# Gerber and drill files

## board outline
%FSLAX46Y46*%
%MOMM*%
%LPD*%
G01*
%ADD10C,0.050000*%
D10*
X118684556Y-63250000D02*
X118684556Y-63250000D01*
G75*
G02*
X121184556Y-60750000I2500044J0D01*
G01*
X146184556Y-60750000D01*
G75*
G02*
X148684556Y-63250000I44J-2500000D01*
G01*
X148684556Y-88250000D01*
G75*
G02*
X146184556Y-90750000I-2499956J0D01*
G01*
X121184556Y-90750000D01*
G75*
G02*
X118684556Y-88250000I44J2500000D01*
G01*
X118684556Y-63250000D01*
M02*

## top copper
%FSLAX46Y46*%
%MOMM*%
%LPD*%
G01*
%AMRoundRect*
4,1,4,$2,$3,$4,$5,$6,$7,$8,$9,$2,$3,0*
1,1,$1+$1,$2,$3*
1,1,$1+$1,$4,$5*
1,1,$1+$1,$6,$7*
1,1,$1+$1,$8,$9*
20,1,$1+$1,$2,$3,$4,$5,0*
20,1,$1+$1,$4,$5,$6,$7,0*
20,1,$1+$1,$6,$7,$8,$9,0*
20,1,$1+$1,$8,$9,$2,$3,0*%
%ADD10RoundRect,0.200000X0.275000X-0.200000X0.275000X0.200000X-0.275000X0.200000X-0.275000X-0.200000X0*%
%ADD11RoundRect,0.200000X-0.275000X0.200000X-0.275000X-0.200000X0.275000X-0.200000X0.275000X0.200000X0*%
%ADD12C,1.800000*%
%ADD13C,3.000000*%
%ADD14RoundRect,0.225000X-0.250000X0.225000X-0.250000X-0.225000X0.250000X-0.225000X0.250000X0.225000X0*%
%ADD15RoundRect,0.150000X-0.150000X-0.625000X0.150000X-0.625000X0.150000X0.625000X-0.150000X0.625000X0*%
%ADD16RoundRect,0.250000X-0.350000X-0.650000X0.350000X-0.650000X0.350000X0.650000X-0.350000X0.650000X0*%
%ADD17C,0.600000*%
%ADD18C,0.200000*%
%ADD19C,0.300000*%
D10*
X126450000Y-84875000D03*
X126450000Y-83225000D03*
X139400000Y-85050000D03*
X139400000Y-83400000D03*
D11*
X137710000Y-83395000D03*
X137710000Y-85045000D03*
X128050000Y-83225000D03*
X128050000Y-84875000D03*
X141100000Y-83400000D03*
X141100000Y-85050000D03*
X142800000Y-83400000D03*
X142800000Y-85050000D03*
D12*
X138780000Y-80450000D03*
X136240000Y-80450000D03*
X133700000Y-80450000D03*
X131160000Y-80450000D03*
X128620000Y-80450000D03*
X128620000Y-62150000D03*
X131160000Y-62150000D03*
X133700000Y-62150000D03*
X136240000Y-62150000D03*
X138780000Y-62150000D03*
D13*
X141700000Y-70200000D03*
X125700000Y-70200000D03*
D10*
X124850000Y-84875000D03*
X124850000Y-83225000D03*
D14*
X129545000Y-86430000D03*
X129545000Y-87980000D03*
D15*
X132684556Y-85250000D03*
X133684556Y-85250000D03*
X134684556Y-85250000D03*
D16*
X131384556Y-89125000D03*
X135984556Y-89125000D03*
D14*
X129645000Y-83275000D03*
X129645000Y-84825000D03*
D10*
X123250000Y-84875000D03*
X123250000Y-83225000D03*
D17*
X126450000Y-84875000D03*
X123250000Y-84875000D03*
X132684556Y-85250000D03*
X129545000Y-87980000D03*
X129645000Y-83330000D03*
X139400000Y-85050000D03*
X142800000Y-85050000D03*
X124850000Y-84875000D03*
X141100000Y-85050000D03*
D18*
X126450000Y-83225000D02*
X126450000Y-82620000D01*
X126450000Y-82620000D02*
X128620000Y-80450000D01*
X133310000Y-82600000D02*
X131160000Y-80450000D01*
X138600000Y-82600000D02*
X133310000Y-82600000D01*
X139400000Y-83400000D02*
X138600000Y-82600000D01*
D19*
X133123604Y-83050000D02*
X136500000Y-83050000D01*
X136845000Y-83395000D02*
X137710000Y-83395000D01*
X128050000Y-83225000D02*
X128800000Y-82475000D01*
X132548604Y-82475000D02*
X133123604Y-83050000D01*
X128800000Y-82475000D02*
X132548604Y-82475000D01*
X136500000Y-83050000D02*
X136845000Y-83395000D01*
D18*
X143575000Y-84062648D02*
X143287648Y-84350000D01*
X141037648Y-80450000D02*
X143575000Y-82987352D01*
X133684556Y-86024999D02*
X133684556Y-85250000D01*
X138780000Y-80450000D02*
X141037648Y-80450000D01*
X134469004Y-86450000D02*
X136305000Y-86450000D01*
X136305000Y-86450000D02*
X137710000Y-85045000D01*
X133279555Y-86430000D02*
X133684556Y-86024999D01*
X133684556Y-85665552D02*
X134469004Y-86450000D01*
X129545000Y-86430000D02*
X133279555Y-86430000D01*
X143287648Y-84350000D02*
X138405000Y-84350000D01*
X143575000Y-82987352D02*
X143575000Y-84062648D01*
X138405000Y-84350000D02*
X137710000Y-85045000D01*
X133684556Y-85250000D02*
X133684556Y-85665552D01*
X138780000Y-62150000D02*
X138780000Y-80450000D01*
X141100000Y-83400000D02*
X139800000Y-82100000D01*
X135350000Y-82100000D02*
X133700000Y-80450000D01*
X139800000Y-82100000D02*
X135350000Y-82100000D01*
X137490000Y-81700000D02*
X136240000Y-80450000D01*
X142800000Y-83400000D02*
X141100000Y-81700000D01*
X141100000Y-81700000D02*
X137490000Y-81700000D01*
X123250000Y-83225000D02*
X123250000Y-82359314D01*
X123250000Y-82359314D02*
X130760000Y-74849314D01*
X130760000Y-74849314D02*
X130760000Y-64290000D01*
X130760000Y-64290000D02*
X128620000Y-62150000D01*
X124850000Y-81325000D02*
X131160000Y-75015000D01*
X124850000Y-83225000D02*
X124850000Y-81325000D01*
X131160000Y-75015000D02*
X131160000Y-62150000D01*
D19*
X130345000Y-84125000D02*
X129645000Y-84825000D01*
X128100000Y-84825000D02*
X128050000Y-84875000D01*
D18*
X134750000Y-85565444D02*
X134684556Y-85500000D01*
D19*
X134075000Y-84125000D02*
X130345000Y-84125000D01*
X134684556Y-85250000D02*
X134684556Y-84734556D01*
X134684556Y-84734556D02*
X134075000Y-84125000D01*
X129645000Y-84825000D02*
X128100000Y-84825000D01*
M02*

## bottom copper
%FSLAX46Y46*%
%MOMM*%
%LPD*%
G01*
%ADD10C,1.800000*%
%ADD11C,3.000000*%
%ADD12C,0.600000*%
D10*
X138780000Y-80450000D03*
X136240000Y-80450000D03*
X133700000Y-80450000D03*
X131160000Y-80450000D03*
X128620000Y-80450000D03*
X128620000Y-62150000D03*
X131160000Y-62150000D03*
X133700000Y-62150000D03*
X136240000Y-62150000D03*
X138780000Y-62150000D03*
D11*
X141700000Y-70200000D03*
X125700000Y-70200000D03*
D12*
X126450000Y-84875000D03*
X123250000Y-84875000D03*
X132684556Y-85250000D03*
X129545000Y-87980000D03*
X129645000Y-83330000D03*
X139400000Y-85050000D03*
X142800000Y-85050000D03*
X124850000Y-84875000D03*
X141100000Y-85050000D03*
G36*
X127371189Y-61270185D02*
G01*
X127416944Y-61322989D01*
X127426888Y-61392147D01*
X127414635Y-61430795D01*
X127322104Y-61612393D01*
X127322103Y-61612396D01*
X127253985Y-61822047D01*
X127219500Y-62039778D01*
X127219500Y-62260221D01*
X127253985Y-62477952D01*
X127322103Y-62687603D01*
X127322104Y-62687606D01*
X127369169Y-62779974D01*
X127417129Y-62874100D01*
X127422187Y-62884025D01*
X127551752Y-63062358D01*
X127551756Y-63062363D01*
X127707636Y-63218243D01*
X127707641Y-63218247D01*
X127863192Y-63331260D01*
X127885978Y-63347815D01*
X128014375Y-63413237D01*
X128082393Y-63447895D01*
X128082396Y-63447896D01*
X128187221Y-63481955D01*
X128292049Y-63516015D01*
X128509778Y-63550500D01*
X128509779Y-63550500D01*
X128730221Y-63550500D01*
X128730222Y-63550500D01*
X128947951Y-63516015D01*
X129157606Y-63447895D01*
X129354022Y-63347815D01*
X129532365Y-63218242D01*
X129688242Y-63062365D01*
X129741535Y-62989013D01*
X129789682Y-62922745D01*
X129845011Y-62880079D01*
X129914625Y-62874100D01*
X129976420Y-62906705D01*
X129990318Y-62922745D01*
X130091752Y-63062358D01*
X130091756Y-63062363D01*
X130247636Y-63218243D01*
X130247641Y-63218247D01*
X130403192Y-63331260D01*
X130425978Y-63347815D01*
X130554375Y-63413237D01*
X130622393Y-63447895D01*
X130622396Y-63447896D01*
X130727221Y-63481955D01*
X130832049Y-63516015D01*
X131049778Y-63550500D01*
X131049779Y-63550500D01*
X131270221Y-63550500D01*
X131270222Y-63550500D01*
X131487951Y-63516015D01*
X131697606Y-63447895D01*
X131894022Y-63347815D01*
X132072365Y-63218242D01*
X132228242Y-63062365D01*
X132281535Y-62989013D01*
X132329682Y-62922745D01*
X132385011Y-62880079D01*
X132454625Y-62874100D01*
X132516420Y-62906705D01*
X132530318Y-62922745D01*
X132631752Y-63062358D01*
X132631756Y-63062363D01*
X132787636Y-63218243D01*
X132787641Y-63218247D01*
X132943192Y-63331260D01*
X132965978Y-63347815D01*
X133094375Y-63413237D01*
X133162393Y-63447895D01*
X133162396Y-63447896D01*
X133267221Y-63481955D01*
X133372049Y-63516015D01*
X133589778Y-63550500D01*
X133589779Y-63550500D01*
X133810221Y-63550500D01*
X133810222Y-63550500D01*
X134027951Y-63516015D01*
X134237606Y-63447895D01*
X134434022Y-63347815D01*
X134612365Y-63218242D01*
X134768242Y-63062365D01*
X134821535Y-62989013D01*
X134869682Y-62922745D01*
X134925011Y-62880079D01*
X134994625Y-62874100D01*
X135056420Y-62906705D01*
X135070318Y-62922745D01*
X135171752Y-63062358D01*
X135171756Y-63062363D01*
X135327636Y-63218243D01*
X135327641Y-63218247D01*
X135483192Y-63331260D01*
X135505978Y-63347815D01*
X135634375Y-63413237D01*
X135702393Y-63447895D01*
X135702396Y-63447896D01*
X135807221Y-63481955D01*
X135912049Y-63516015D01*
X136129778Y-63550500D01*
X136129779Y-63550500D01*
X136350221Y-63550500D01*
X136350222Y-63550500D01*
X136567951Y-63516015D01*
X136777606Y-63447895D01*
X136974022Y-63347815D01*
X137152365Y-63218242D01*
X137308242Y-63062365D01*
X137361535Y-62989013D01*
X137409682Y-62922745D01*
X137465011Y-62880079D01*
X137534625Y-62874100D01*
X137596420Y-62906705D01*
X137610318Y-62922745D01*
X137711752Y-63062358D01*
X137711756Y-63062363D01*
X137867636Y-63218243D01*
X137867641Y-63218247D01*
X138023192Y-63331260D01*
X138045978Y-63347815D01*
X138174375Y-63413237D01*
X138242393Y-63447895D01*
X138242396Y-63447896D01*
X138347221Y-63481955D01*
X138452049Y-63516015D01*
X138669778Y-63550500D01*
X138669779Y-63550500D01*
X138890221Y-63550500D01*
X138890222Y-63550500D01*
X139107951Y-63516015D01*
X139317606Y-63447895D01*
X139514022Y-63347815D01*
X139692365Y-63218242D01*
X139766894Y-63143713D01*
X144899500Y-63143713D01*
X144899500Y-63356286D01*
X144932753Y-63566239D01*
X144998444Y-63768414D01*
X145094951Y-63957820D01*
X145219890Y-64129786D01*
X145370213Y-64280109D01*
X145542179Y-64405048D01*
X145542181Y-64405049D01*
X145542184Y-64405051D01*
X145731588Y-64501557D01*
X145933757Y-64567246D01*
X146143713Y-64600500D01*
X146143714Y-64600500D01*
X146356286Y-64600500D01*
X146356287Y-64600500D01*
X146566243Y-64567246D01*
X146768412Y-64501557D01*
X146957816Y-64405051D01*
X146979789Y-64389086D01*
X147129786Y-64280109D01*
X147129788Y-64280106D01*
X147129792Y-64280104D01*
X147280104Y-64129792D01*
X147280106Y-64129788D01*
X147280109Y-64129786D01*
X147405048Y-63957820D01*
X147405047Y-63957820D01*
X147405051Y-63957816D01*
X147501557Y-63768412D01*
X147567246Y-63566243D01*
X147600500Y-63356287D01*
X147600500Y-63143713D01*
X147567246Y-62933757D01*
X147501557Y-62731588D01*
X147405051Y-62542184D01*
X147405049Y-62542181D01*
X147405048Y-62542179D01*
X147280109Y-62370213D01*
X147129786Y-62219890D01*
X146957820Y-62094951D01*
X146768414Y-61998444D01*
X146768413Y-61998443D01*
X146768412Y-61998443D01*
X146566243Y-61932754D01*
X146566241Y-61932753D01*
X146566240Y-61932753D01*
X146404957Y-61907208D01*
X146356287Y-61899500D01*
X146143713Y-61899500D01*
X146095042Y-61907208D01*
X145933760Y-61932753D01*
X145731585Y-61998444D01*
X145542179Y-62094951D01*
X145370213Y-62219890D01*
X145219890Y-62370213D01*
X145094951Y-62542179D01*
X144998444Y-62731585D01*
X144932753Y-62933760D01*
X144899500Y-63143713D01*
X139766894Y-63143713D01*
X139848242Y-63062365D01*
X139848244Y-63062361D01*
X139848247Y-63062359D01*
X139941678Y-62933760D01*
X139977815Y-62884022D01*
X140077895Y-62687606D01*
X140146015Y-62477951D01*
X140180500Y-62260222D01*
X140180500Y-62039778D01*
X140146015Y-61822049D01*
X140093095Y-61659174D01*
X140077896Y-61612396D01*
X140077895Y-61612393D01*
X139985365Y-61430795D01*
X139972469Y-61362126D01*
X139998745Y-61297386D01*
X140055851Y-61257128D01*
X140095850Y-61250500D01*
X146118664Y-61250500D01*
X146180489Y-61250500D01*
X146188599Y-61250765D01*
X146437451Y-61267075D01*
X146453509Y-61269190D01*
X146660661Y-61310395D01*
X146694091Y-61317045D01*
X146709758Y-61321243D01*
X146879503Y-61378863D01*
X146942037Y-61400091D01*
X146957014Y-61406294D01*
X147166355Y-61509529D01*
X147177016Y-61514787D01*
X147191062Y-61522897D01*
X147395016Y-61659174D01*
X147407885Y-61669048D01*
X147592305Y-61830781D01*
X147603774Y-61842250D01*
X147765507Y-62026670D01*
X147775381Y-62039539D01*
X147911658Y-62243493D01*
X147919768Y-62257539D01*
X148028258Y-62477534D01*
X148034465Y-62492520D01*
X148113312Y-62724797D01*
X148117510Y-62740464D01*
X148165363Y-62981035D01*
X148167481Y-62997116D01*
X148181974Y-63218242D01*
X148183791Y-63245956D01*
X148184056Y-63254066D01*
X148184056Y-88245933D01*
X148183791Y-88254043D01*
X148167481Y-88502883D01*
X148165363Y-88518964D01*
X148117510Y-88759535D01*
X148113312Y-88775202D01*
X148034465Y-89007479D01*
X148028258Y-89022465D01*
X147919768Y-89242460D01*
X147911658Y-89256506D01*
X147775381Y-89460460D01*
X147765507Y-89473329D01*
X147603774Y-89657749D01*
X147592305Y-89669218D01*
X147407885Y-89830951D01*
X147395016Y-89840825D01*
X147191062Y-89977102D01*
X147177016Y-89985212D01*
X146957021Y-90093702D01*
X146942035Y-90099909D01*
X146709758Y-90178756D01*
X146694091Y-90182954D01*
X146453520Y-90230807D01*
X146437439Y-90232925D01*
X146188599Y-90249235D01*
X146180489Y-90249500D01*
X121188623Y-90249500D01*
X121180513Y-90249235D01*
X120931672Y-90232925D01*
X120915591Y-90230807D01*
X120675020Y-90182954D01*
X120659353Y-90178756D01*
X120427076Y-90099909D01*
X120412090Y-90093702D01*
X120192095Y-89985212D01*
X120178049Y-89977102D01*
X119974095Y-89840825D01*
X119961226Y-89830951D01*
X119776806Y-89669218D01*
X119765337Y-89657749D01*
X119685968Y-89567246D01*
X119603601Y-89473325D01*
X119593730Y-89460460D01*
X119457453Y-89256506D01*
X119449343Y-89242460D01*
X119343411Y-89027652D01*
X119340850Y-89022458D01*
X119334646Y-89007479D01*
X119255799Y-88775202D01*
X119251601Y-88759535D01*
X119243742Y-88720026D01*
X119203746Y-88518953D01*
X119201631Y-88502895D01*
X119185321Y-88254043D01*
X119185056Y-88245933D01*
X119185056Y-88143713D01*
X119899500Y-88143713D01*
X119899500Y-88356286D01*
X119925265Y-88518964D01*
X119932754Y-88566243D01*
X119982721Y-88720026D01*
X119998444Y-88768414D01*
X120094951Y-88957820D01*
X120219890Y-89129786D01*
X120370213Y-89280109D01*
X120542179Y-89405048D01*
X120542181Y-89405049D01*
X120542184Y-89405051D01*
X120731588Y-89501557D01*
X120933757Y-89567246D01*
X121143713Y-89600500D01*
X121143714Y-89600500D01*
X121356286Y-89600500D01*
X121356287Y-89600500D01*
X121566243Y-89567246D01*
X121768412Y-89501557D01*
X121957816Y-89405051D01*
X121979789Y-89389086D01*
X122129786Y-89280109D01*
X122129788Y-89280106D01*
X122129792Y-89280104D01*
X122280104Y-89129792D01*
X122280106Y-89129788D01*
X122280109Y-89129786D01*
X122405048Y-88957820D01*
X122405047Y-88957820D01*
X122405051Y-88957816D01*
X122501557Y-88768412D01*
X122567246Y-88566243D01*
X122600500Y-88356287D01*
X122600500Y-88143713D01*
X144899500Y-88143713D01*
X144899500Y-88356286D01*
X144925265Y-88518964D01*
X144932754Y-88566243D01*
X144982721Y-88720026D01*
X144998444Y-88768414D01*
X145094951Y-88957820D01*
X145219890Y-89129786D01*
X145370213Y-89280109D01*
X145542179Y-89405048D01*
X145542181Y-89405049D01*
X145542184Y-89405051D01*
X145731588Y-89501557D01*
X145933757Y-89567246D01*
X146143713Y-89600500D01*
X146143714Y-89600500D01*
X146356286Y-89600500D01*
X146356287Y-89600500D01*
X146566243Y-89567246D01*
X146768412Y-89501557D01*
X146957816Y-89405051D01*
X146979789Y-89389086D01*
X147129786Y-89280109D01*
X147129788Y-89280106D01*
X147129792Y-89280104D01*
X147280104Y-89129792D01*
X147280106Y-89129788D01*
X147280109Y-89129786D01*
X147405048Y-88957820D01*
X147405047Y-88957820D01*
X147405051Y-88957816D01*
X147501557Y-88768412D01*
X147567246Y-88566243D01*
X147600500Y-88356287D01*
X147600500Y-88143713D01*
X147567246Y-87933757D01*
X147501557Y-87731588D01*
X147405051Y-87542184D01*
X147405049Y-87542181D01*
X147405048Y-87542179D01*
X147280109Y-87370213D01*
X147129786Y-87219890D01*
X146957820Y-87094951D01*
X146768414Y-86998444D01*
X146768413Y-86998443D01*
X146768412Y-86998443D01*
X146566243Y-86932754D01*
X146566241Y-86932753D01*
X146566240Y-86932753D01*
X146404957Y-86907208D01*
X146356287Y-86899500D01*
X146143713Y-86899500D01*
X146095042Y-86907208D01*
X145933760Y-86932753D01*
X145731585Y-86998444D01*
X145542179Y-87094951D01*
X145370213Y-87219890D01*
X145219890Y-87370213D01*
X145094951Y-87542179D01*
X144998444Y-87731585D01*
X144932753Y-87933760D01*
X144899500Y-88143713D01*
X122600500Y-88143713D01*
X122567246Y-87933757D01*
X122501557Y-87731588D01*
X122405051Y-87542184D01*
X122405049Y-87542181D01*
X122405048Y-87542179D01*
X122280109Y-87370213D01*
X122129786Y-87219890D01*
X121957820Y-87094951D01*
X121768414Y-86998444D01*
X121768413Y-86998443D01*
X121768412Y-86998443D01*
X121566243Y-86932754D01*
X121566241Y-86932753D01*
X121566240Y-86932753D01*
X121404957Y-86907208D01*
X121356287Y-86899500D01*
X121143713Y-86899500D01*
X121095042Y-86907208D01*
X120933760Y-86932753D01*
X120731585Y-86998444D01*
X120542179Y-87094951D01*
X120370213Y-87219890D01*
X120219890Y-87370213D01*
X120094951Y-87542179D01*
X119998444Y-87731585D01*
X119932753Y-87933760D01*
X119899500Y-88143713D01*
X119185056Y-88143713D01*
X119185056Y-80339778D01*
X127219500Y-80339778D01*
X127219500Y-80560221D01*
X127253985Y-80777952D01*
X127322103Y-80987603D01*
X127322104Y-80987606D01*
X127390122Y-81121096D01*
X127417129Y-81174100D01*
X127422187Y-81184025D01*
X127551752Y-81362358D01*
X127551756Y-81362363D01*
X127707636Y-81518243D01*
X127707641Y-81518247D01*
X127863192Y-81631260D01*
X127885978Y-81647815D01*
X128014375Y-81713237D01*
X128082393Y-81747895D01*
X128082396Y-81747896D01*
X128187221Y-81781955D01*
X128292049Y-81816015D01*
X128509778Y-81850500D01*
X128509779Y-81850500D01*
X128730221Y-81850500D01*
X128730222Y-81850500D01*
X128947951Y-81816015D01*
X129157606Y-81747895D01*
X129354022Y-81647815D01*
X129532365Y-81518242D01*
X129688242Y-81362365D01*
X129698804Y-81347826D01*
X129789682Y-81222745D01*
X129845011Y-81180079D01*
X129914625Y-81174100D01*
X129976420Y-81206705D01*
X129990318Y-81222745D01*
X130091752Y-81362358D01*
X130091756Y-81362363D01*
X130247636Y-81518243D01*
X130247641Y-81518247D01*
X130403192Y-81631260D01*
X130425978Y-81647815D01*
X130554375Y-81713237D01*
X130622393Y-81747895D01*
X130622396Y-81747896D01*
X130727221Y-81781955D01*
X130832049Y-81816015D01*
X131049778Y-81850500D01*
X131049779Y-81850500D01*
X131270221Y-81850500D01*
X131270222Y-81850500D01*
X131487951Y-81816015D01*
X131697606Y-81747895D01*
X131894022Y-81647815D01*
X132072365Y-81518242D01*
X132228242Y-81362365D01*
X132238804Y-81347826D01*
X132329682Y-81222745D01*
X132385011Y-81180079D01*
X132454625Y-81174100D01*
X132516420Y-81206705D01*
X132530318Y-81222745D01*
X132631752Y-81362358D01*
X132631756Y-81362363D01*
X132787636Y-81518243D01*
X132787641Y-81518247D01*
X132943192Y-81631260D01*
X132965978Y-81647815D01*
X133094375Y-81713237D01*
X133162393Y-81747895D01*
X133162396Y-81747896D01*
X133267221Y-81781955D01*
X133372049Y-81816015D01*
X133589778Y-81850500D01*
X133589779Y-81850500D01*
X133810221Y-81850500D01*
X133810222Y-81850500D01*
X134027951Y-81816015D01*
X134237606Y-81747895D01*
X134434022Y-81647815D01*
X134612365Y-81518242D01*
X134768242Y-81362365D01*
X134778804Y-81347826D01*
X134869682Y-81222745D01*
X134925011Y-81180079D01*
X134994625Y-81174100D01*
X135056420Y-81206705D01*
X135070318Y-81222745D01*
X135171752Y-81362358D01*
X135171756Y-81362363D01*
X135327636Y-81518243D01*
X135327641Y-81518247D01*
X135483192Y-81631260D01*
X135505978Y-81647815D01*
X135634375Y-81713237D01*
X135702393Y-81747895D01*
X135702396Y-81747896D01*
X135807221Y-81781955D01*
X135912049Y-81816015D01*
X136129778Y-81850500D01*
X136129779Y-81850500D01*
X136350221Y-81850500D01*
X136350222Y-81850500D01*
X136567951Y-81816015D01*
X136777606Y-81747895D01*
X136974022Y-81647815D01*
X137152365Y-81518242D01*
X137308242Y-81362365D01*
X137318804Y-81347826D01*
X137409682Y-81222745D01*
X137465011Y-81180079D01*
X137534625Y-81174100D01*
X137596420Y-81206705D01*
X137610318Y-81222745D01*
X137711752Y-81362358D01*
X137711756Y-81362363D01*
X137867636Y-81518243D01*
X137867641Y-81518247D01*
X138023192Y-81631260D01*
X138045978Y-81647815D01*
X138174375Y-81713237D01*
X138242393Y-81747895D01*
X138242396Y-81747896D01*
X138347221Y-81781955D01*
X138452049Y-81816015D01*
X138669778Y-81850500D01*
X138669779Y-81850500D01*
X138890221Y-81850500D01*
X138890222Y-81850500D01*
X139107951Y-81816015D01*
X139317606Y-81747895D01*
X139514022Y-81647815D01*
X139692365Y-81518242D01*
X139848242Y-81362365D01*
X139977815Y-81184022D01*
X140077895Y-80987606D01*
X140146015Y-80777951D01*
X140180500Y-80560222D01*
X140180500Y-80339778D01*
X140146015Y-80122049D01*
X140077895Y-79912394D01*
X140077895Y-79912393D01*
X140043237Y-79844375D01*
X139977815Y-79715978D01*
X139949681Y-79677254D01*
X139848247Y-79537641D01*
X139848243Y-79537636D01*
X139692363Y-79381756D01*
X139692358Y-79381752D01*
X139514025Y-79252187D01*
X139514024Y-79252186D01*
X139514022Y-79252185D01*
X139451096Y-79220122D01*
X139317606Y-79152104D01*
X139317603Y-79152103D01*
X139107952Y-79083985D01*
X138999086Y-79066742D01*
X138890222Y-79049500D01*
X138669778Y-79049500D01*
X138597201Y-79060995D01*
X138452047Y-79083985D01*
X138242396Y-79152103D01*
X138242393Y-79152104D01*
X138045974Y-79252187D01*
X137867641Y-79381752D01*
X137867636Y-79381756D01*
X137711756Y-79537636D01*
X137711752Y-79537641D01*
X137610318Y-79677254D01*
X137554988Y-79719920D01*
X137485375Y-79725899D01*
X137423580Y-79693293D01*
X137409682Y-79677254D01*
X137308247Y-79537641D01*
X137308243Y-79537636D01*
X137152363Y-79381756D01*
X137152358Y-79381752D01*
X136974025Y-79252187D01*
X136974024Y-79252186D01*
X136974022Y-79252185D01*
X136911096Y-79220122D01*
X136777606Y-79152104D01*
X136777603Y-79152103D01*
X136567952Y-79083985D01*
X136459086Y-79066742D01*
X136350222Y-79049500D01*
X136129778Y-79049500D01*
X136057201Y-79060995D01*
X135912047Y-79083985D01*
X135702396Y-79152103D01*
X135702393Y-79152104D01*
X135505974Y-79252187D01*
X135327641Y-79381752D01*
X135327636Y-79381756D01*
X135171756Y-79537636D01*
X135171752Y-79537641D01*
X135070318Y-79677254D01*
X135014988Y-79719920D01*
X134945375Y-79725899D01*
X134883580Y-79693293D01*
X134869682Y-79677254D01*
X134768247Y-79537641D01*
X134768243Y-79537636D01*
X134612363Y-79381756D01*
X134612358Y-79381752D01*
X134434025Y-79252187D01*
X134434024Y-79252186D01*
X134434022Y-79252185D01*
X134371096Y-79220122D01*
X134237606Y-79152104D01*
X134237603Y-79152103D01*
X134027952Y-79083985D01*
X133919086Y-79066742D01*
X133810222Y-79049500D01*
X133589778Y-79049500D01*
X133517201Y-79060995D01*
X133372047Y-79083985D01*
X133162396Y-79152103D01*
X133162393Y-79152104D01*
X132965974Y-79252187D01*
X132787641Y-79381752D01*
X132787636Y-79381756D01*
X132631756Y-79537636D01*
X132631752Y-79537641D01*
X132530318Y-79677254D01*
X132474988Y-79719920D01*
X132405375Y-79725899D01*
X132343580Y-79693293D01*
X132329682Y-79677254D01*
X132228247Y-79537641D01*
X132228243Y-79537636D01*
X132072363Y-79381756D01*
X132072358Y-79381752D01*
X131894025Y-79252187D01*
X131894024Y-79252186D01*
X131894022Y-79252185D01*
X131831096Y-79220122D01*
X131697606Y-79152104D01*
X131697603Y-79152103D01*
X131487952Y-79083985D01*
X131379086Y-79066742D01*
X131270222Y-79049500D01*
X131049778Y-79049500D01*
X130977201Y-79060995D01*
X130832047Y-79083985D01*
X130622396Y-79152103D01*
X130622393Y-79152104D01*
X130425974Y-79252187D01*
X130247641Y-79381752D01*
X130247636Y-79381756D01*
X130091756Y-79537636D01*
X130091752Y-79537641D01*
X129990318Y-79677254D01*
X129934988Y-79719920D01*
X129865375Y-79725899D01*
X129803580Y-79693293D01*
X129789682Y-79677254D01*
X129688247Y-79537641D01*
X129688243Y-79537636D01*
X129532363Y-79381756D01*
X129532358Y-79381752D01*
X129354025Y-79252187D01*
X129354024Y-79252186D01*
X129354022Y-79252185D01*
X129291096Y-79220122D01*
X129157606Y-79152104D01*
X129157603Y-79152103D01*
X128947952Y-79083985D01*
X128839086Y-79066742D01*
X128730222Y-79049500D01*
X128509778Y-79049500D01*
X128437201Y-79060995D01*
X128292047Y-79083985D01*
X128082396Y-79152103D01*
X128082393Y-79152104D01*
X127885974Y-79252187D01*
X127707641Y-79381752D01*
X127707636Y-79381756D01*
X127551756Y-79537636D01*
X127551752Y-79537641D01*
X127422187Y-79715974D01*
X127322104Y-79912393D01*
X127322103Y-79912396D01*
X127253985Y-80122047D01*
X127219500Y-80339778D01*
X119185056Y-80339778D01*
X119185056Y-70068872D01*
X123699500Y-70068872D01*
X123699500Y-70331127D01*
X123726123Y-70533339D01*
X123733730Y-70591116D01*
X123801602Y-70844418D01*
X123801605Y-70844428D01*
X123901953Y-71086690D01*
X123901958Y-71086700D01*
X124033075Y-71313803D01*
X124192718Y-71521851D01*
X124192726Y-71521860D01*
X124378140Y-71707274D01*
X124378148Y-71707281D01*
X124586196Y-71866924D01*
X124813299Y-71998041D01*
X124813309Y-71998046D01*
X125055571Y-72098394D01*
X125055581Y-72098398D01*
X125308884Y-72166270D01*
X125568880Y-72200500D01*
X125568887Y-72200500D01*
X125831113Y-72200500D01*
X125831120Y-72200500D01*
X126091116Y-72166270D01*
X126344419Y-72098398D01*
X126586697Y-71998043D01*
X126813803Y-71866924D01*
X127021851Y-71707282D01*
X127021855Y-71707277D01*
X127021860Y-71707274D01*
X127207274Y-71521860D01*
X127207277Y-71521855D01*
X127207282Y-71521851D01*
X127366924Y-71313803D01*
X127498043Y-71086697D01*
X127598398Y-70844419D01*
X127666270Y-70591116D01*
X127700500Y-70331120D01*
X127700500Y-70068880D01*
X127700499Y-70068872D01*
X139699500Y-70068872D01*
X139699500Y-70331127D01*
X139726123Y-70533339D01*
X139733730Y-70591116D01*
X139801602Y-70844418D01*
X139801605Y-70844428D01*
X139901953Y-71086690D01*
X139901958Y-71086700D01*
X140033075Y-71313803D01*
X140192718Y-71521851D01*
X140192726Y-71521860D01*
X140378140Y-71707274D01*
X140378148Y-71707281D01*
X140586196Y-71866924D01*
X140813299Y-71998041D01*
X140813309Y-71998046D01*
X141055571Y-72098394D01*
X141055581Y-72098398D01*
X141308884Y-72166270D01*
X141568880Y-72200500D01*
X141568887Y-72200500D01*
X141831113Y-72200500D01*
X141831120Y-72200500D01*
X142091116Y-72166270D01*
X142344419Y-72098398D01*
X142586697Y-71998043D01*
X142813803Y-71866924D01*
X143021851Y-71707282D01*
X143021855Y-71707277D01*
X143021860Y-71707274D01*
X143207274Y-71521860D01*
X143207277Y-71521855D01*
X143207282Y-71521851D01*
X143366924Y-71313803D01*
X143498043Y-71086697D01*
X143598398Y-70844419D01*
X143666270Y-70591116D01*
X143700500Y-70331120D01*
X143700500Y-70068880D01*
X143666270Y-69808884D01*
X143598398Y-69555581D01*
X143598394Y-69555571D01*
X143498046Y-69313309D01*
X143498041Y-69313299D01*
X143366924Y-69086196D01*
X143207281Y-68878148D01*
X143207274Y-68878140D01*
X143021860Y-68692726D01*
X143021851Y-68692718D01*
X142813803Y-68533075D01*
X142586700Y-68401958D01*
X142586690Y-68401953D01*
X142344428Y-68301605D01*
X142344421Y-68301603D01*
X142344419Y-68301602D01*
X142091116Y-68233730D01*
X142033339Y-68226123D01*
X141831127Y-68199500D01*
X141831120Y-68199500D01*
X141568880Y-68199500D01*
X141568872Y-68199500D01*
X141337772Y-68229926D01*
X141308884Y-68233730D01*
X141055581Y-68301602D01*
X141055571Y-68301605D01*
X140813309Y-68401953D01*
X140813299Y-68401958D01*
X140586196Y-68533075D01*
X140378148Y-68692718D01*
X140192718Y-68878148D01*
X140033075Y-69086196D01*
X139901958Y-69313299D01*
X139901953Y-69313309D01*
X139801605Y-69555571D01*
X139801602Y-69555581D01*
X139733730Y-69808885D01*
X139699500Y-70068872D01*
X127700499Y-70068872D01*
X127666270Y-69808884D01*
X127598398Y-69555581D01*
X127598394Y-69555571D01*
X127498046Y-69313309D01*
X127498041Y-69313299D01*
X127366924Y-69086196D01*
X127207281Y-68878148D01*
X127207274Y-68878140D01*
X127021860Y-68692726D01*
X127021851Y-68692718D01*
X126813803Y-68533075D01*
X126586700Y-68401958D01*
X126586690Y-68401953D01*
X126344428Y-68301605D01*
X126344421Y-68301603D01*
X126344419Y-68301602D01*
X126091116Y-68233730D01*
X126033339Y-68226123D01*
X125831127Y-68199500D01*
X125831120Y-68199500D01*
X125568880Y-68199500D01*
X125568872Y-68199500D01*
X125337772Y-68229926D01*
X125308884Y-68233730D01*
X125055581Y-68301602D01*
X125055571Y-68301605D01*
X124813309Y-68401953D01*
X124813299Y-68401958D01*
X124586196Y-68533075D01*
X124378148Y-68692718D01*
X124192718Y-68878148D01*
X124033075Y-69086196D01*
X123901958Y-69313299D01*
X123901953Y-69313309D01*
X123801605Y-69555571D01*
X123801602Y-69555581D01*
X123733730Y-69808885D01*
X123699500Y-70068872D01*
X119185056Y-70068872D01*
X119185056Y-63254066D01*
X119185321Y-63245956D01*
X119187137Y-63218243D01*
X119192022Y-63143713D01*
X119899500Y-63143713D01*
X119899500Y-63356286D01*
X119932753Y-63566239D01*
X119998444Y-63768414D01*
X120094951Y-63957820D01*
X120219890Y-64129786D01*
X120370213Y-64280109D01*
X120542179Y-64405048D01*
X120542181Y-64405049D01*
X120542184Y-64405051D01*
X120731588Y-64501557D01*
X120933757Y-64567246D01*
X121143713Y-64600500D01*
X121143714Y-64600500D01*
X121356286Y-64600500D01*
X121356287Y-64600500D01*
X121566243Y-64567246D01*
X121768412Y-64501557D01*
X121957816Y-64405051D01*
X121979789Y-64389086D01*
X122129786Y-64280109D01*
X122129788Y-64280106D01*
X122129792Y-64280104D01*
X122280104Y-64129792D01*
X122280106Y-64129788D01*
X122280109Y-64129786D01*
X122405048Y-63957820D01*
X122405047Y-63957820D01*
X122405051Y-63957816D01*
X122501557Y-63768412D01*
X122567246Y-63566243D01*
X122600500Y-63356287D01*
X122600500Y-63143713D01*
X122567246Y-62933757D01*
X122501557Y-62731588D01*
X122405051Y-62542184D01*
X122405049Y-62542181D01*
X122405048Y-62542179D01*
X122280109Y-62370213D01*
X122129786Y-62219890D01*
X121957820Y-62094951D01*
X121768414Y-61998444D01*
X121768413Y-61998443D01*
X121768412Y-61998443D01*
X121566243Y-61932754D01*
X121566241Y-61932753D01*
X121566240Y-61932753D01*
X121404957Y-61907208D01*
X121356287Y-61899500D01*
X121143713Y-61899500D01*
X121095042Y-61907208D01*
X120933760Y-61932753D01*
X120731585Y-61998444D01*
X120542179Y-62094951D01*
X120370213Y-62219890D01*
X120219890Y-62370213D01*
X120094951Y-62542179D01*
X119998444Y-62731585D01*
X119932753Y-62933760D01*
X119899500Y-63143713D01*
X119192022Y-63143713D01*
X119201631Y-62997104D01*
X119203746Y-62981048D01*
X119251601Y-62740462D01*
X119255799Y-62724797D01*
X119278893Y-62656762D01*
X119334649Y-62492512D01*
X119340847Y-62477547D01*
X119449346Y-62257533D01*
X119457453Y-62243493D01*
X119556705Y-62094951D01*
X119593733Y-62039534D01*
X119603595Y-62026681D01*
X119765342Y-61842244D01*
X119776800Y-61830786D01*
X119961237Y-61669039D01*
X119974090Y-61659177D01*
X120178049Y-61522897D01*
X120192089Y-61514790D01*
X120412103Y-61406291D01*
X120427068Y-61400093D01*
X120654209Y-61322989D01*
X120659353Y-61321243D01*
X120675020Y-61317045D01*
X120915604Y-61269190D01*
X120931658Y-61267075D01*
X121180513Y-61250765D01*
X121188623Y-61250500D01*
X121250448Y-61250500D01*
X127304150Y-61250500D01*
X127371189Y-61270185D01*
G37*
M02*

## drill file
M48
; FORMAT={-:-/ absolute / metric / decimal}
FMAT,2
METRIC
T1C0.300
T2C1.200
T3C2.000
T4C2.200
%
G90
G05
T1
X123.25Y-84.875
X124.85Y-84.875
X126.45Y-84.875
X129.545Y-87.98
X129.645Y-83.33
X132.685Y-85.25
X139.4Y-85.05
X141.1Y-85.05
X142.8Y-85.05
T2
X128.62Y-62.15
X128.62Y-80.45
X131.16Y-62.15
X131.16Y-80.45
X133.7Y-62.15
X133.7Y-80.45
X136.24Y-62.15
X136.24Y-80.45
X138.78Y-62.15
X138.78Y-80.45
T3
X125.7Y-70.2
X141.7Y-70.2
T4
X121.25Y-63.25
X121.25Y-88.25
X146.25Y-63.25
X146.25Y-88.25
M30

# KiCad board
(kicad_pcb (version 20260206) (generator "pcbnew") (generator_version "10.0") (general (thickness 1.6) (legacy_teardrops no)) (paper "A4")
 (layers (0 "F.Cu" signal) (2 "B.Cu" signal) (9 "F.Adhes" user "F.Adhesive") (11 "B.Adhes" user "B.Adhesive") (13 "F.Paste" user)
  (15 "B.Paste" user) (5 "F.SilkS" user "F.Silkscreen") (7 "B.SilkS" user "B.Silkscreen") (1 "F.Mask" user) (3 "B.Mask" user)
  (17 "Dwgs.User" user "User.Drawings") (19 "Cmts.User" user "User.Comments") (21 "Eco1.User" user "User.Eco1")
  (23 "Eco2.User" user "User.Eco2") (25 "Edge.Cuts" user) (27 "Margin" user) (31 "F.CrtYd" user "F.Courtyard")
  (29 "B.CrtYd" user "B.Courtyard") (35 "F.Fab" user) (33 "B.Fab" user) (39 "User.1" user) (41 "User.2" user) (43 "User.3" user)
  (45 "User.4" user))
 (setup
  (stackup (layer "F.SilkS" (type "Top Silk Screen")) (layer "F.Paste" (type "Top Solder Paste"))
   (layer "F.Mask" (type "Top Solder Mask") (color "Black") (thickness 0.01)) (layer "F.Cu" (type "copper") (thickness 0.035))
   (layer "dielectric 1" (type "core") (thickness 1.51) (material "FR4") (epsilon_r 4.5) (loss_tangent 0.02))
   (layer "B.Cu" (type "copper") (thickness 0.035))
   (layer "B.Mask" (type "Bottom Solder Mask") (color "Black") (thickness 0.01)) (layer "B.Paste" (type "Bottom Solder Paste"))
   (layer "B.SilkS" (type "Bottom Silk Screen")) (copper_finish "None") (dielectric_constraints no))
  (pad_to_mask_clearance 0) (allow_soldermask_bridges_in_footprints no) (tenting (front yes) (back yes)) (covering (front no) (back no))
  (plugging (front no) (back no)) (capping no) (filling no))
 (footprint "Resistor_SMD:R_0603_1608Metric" (layer "F.Cu") (at 126.45 84.05 90)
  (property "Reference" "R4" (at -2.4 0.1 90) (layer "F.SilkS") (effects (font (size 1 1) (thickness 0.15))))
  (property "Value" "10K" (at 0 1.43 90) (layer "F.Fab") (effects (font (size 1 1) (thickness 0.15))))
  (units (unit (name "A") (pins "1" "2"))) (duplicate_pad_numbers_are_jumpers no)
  (pad "1" smd roundrect (at -0.825 0 90) (size 0.8 0.95) (layers "F.Cu" "F.Mask" "F.Paste") (roundrect_rratio 0.25) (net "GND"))
  (pad "2" smd roundrect (at 0.825 0 90) (size 0.8 0.95) (layers "F.Cu" "F.Mask" "F.Paste") (roundrect_rratio 0.25) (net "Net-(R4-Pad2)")))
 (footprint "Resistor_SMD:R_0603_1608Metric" (layer "F.Cu") (at 139.4 84.225 90)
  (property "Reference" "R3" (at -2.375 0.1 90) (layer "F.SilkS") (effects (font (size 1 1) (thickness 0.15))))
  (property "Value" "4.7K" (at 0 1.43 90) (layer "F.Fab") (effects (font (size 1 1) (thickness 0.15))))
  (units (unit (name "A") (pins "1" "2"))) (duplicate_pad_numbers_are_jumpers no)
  (pad "1" smd roundrect (at -0.825 0 90) (size 0.8 0.95) (layers "F.Cu" "F.Mask" "F.Paste") (roundrect_rratio 0.25) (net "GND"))
  (pad "2" smd roundrect (at 0.825 0 90) (size 0.8 0.95) (layers "F.Cu" "F.Mask" "F.Paste") (roundrect_rratio 0.25) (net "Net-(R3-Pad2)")))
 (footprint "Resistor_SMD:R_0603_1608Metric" (layer "F.Cu") (at 137.71 84.22 -90)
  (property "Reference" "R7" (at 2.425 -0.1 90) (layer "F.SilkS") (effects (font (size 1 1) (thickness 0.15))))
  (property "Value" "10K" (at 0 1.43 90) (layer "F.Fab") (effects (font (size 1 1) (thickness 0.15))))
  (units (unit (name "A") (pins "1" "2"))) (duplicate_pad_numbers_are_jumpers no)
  (pad "1" smd roundrect (at -0.825 0 270) (size 0.8 0.95) (layers "F.Cu" "F.Mask" "F.Paste") (roundrect_rratio 0.25) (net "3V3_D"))
  (pad "2" smd roundrect (at 0.825 0 270) (size 0.8 0.95) (layers "F.Cu" "F.Mask" "F.Paste") (roundrect_rratio 0.25) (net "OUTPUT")))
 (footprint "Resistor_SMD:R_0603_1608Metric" (layer "F.Cu") (at 128.05 84.05 -90)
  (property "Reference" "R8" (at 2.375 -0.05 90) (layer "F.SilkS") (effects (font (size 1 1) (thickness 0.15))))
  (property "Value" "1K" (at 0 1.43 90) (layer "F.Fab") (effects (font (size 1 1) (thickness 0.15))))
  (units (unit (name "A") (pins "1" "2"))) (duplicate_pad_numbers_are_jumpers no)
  (pad "1" smd roundrect (at -0.825 0 270) (size 0.8 0.95) (layers "F.Cu" "F.Mask" "F.Paste") (roundrect_rratio 0.25) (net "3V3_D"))
  (pad "2" smd roundrect (at 0.825 0 270) (size 0.8 0.95) (layers "F.Cu" "F.Mask" "F.Paste") (roundrect_rratio 0.25) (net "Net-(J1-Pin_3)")))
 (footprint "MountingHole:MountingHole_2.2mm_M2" (layer "F.Cu") (at 146.25 63.25)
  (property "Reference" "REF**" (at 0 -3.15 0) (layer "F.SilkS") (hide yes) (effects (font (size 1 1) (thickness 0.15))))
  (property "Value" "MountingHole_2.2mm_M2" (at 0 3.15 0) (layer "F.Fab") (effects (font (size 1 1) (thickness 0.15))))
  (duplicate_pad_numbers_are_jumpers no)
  (pad "" np_thru_hole circle (at 0 0) (size 2.2 2.2) (drill 2.2) (layers "*.Cu" "*.Mask")))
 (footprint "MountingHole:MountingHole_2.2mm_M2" (layer "F.Cu") (at 146.25 88.25)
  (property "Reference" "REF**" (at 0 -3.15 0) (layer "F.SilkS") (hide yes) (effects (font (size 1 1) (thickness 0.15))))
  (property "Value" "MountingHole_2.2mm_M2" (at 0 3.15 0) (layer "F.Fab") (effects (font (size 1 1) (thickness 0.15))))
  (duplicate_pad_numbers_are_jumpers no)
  (pad "" np_thru_hole circle (at 0 0) (size 2.2 2.2) (drill 2.2) (layers "*.Cu" "*.Mask")))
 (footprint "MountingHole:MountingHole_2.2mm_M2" (layer "F.Cu") (at 121.25 88.25)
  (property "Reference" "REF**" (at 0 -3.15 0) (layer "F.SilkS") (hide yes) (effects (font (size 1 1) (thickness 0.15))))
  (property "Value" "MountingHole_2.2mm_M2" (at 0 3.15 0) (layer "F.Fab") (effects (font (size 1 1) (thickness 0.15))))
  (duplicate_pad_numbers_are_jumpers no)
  (pad "" np_thru_hole circle (at 0 0) (size 2.2 2.2) (drill 2.2) (layers "*.Cu" "*.Mask")))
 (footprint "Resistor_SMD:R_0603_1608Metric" (layer "F.Cu") (at 141.1 84.225 -90)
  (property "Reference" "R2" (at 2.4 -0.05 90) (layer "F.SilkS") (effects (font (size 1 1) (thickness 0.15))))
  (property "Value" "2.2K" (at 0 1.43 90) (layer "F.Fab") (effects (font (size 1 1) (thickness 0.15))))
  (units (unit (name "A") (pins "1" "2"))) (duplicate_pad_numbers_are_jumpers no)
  (pad "1" smd roundrect (at -0.825 0 270) (size 0.8 0.95) (layers "F.Cu" "F.Mask" "F.Paste") (roundrect_rratio 0.25) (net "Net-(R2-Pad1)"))
  (pad "2" smd roundrect (at 0.825 0 270) (size 0.8 0.95) (layers "F.Cu" "F.Mask" "F.Paste") (roundrect_rratio 0.25) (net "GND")))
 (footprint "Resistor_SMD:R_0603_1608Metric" (layer "F.Cu") (at 142.8 84.225 -90)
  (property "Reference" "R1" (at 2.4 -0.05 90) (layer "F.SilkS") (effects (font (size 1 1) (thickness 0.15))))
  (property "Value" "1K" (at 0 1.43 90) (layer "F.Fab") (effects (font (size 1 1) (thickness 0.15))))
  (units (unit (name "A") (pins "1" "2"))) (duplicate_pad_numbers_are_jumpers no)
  (pad "1" smd roundrect (at -0.825 0 270) (size 0.8 0.95) (layers "F.Cu" "F.Mask" "F.Paste") (roundrect_rratio 0.25) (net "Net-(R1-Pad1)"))
  (pad "2" smd roundrect (at 0.825 0 270) (size 0.8 0.95) (layers "F.Cu" "F.Mask" "F.Paste") (roundrect_rratio 0.25) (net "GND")))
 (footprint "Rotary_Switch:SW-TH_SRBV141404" (layer "F.Cu") (at 133.7 71.3)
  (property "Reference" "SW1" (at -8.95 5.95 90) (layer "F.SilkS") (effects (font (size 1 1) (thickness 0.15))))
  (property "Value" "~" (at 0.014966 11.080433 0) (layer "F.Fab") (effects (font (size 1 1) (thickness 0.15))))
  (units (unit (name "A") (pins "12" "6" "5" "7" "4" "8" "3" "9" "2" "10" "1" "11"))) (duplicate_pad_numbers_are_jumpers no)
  (pad "1" thru_hole circle (at 5.08 9.15) (size 1.8 1.8) (drill 1.2) (layers "*.Cu" "*.Mask") (remove_unused_layers no) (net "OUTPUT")
   (thermal_bridge_angle 90))
  (pad "2" thru_hole circle (at 2.54 9.15) (size 1.8 1.8) (drill 1.2) (layers "*.Cu" "*.Mask") (remove_unused_layers no)
   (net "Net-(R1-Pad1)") (thermal_bridge_angle 90))
  (pad "3" thru_hole circle (at 0 9.15) (size 1.8 1.8) (drill 1.2) (layers "*.Cu" "*.Mask") (remove_unused_layers no) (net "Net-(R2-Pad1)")
   (thermal_bridge_angle 90))
  (pad "4" thru_hole circle (at -2.54 9.15) (size 1.8 1.8) (drill 1.2) (layers "*.Cu" "*.Mask") (remove_unused_layers no)
   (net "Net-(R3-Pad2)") (thermal_bridge_angle 90))
  (pad "5" thru_hole circle (at -5.08 9.15) (size 1.8 1.8) (drill 1.2) (layers "*.Cu" "*.Mask") (remove_unused_layers no)
   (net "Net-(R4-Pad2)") (thermal_bridge_angle 90))
  (pad "6" thru_hole circle (at -5.08 -9.15) (size 1.8 1.8) (drill 1.2) (layers "*.Cu" "*.Mask") (remove_unused_layers no)
   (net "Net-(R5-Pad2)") (thermal_bridge_angle 90))
  (pad "7" thru_hole circle (at -2.54 -9.15) (size 1.8 1.8) (drill 1.2) (layers "*.Cu" "*.Mask") (remove_unused_layers no)
   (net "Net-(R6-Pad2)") (thermal_bridge_angle 90))
  (pad "8" thru_hole circle (at 0 -9.15) (size 1.8 1.8) (drill 1.2) (layers "*.Cu" "*.Mask") (remove_unused_layers no)
   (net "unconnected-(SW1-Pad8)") (thermal_bridge_angle 90))
  (pad "9" thru_hole circle (at 2.54 -9.15) (size 1.8 1.8) (drill 1.2) (layers "*.Cu" "*.Mask") (remove_unused_layers no)
   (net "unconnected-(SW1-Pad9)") (thermal_bridge_angle 90))
  (pad "10" thru_hole circle (at 5.08 -9.15) (size 1.8 1.8) (drill 1.2) (layers "*.Cu" "*.Mask") (remove_unused_layers no) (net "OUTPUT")
   (thermal_bridge_angle 90))
  (pad "11" thru_hole circle (at 8 -1.1) (size 3 3) (drill 2) (layers "*.Cu" "*.Mask") (remove_unused_layers no)
   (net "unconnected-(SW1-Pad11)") (thermal_bridge_angle 90))
  (pad "12" thru_hole circle (at -8 -1.1) (size 3 3) (drill 2) (layers "*.Cu" "*.Mask") (remove_unused_layers no)
   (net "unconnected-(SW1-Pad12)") (thermal_bridge_angle 90)))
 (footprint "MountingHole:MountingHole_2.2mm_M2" (layer "F.Cu") (at 121.25 63.25)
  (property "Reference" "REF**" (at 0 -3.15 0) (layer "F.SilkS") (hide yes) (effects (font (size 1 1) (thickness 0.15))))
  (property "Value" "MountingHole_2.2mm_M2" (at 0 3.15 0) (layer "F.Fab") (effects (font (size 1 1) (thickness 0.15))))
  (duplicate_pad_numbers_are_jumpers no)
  (pad "" np_thru_hole circle (at 0 0) (size 2.2 2.2) (drill 2.2) (layers "*.Cu" "*.Mask")))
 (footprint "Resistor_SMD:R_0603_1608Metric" (layer "F.Cu") (at 124.85 84.05 90)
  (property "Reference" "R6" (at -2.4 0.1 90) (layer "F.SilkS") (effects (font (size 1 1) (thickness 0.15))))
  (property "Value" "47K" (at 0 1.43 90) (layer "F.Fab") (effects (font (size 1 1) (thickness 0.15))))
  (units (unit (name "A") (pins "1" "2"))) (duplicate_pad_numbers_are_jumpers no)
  (pad "1" smd roundrect (at -0.825 0 90) (size 0.8 0.95) (layers "F.Cu" "F.Mask" "F.Paste") (roundrect_rratio 0.25) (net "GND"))
  (pad "2" smd roundrect (at 0.825 0 90) (size 0.8 0.95) (layers "F.Cu" "F.Mask" "F.Paste") (roundrect_rratio 0.25) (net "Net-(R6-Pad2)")))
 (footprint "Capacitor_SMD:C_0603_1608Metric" (layer "F.Cu") (at 129.545 87.205 -90)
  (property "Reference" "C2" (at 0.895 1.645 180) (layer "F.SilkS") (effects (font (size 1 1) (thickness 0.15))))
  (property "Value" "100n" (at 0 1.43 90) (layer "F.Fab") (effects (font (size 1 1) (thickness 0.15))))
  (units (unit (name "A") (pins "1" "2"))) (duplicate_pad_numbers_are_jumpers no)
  (pad "1" smd roundrect (at -0.775 0 270) (size 0.9 0.95) (layers "F.Cu" "F.Mask" "F.Paste") (roundrect_rratio 0.25) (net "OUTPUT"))
  (pad "2" smd roundrect (at 0.775 0 270) (size 0.9 0.95) (layers "F.Cu" "F.Mask" "F.Paste") (roundrect_rratio 0.25) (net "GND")))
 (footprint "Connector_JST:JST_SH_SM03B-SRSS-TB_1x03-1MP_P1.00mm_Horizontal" (layer "F.Cu") (at 133.684556 87.25)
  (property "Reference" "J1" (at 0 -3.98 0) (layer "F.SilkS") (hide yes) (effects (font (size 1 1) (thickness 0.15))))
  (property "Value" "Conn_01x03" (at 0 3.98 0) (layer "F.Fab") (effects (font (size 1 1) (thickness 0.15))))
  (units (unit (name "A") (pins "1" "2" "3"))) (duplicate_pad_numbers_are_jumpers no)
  (pad "1" smd roundrect (at -1 -2) (size 0.6 1.55) (layers "F.Cu" "F.Mask" "F.Paste") (roundrect_rratio 0.25) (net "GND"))
  (pad "2" smd roundrect (at 0 -2) (size 0.6 1.55) (layers "F.Cu" "F.Mask" "F.Paste") (roundrect_rratio 0.25) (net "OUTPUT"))
  (pad "3" smd roundrect (at 1 -2) (size 0.6 1.55) (layers "F.Cu" "F.Mask" "F.Paste") (roundrect_rratio 0.25) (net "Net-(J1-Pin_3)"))
  (pad "MP" smd roundrect (at -2.3 1.875) (size 1.2 1.8) (layers "F.Cu" "F.Mask" "F.Paste") (roundrect_rratio 0.208333))
  (pad "MP" smd roundrect (at 2.3 1.875) (size 1.2 1.8) (layers "F.Cu" "F.Mask" "F.Paste") (roundrect_rratio 0.208333)))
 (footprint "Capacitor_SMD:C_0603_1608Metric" (layer "F.Cu") (at 129.645 84.05 -90)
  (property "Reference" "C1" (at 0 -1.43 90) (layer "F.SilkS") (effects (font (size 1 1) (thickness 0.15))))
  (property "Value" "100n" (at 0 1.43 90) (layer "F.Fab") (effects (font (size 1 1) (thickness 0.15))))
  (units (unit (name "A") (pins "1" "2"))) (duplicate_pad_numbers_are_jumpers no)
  (pad "1" smd roundrect (at -0.775 0 270) (size 0.9 0.95) (layers "F.Cu" "F.Mask" "F.Paste") (roundrect_rratio 0.25) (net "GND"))
  (pad "2" smd roundrect (at 0.775 0 270) (size 0.9 0.95) (layers "F.Cu" "F.Mask" "F.Paste") (roundrect_rratio 0.25) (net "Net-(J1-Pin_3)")))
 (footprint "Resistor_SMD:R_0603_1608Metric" (layer "F.Cu") (at 123.25 84.05 90)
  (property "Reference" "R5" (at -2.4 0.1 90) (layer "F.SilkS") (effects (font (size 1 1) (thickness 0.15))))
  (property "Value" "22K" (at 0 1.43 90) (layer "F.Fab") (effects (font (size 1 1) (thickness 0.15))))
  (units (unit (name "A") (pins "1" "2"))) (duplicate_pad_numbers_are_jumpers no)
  (pad "1" smd roundrect (at -0.825 0 90) (size 0.8 0.95) (layers "F.Cu" "F.Mask" "F.Paste") (roundrect_rratio 0.25) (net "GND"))
  (pad "2" smd roundrect (at 0.825 0 90) (size 0.8 0.95) (layers "F.Cu" "F.Mask" "F.Paste") (roundrect_rratio 0.25) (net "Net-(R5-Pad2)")))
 (gr_rect (start 118.684556 60.75) (end 148.684556 90.75) (radius 2.5) (stroke (width 0.05) (type solid)) (fill no) (layer "Edge.Cuts"))
 (via (at 126.45 84.875) (size 0.6) (drill 0.3) (layers "F.Cu" "B.Cu") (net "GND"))
 (via (at 123.25 84.875) (size 0.6) (drill 0.3) (layers "F.Cu" "B.Cu") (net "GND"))
 (via (at 132.684556 85.25) (size 0.6) (drill 0.3) (layers "F.Cu" "B.Cu") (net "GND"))
 (via (at 129.545 87.98) (size 0.6) (drill 0.3) (layers "F.Cu" "B.Cu") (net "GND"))
 (via (at 129.645 83.33) (size 0.6) (drill 0.3) (layers "F.Cu" "B.Cu") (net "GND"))
 (via (at 139.4 85.05) (size 0.6) (drill 0.3) (layers "F.Cu" "B.Cu") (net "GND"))
 (via (at 142.8 85.05) (size 0.6) (drill 0.3) (layers "F.Cu" "B.Cu") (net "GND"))
 (via (at 124.85 84.875) (size 0.6) (drill 0.3) (layers "F.Cu" "B.Cu") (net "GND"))
 (via (at 141.1 85.05) (size 0.6) (drill 0.3) (layers "F.Cu" "B.Cu") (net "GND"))
 (segment (start 126.45 83.225) (end 126.45 82.62) (width 0.2) (layer "F.Cu") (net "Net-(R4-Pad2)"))
 (segment (start 126.45 82.62) (end 128.62 80.45) (width 0.2) (layer "F.Cu") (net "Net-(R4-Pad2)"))
 (segment (start 133.31 82.6) (end 131.16 80.45) (width 0.2) (layer "F.Cu") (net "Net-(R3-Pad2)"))
 (segment (start 138.6 82.6) (end 133.31 82.6) (width 0.2) (layer "F.Cu") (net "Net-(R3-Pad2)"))
 (segment (start 139.4 83.4) (end 138.6 82.6) (width 0.2) (layer "F.Cu") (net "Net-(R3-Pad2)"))
 (segment (start 133.123604 83.05) (end 136.5 83.05) (width 0.3) (layer "F.Cu") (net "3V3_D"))
 (segment (start 136.845 83.395) (end 137.71 83.395) (width 0.3) (layer "F.Cu") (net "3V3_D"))
 (segment (start 128.05 83.225) (end 128.8 82.475) (width 0.3) (layer "F.Cu") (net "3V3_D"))
 (segment (start 132.548604 82.475) (end 133.123604 83.05) (width 0.3) (layer "F.Cu") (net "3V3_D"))
 (segment (start 128.8 82.475) (end 132.548604 82.475) (width 0.3) (layer "F.Cu") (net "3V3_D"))
 (segment (start 136.5 83.05) (end 136.845 83.395) (width 0.3) (layer "F.Cu") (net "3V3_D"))
 (segment (start 143.575 84.062648) (end 143.287648 84.35) (width 0.2) (layer "F.Cu") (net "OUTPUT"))
 (segment (start 141.037648 80.45) (end 143.575 82.987352) (width 0.2) (layer "F.Cu") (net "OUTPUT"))
 (segment (start 133.684556 86.024999) (end 133.684556 85.25) (width 0.2) (layer "F.Cu") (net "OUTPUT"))
 (segment (start 138.78 80.45) (end 141.037648 80.45) (width 0.2) (layer "F.Cu") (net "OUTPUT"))
 (segment (start 134.469004 86.45) (end 136.305 86.45) (width 0.2) (layer "F.Cu") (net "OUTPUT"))
 (segment (start 136.305 86.45) (end 137.71 85.045) (width 0.2) (layer "F.Cu") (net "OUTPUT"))
 (segment (start 133.279555 86.43) (end 133.684556 86.024999) (width 0.2) (layer "F.Cu") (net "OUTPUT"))
 (segment (start 133.684556 85.665552) (end 134.469004 86.45) (width 0.2) (layer "F.Cu") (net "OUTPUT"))
 (segment (start 129.545 86.43) (end 133.279555 86.43) (width 0.2) (layer "F.Cu") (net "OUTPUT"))
 (segment (start 143.287648 84.35) (end 138.405 84.35) (width 0.2) (layer "F.Cu") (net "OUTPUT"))
 (segment (start 143.575 82.987352) (end 143.575 84.062648) (width 0.2) (layer "F.Cu") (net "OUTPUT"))
 (segment (start 138.405 84.35) (end 137.71 85.045) (width 0.2) (layer "F.Cu") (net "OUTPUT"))
 (segment (start 133.684556 85.25) (end 133.684556 85.665552) (width 0.2) (layer "F.Cu") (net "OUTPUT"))
 (segment (start 138.78 62.15) (end 138.78 80.45) (width 0.2) (layer "F.Cu") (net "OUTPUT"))
 (segment (start 141.1 83.4) (end 139.8 82.1) (width 0.2) (layer "F.Cu") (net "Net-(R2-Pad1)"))
 (segment (start 135.35 82.1) (end 133.7 80.45) (width 0.2) (layer "F.Cu") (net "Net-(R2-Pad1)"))
 (segment (start 139.8 82.1) (end 135.35 82.1) (width 0.2) (layer "F.Cu") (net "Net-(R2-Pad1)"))
 (segment (start 137.49 81.7) (end 136.24 80.45) (width 0.2) (layer "F.Cu") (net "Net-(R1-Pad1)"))
 (segment (start 142.8 83.4) (end 141.1 81.7) (width 0.2) (layer "F.Cu") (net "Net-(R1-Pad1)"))
 (segment (start 141.1 81.7) (end 137.49 81.7) (width 0.2) (layer "F.Cu") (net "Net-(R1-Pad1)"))
 (segment (start 123.25 83.225) (end 123.25 82.359314) (width 0.2) (layer "F.Cu") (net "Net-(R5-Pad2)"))
 (segment (start 123.25 82.359314) (end 130.76 74.849314) (width 0.2) (layer "F.Cu") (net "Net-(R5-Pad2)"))
 (segment (start 130.76 74.849314) (end 130.76 64.29) (width 0.2) (layer "F.Cu") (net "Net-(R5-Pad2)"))
 (segment (start 130.76 64.29) (end 128.62 62.15) (width 0.2) (layer "F.Cu") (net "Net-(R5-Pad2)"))
 (segment (start 124.85 81.325) (end 131.16 75.015) (width 0.2) (layer "F.Cu") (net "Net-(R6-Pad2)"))
 (segment (start 124.85 83.225) (end 124.85 81.325) (width 0.2) (layer "F.Cu") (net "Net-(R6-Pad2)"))
 (segment (start 131.16 75.015) (end 131.16 62.15) (width 0.2) (layer "F.Cu") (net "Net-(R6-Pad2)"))
 (segment (start 130.345 84.125) (end 129.645 84.825) (width 0.3) (layer "F.Cu") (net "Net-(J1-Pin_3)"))
 (segment (start 128.1 84.825) (end 128.05 84.875) (width 0.3) (layer "F.Cu") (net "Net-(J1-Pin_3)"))
 (segment (start 134.75 85.565444) (end 134.684556 85.5) (width 0.2) (layer "F.Cu") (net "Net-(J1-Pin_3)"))
 (segment (start 134.075 84.125) (end 130.345 84.125) (width 0.3) (layer "F.Cu") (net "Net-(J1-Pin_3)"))
 (segment (start 134.684556 85.25) (end 134.684556 84.734556) (width 0.3) (layer "F.Cu") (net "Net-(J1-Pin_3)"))
 (segment (start 134.684556 84.734556) (end 134.075 84.125) (width 0.3) (layer "F.Cu") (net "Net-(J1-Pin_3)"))
 (segment (start 129.645 84.825) (end 128.1 84.825) (width 0.3) (layer "F.Cu") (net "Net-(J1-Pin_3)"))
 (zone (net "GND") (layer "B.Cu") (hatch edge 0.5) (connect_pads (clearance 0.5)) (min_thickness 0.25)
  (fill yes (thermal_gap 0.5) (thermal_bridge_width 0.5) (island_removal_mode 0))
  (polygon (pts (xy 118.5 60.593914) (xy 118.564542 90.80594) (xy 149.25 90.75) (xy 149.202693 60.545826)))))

